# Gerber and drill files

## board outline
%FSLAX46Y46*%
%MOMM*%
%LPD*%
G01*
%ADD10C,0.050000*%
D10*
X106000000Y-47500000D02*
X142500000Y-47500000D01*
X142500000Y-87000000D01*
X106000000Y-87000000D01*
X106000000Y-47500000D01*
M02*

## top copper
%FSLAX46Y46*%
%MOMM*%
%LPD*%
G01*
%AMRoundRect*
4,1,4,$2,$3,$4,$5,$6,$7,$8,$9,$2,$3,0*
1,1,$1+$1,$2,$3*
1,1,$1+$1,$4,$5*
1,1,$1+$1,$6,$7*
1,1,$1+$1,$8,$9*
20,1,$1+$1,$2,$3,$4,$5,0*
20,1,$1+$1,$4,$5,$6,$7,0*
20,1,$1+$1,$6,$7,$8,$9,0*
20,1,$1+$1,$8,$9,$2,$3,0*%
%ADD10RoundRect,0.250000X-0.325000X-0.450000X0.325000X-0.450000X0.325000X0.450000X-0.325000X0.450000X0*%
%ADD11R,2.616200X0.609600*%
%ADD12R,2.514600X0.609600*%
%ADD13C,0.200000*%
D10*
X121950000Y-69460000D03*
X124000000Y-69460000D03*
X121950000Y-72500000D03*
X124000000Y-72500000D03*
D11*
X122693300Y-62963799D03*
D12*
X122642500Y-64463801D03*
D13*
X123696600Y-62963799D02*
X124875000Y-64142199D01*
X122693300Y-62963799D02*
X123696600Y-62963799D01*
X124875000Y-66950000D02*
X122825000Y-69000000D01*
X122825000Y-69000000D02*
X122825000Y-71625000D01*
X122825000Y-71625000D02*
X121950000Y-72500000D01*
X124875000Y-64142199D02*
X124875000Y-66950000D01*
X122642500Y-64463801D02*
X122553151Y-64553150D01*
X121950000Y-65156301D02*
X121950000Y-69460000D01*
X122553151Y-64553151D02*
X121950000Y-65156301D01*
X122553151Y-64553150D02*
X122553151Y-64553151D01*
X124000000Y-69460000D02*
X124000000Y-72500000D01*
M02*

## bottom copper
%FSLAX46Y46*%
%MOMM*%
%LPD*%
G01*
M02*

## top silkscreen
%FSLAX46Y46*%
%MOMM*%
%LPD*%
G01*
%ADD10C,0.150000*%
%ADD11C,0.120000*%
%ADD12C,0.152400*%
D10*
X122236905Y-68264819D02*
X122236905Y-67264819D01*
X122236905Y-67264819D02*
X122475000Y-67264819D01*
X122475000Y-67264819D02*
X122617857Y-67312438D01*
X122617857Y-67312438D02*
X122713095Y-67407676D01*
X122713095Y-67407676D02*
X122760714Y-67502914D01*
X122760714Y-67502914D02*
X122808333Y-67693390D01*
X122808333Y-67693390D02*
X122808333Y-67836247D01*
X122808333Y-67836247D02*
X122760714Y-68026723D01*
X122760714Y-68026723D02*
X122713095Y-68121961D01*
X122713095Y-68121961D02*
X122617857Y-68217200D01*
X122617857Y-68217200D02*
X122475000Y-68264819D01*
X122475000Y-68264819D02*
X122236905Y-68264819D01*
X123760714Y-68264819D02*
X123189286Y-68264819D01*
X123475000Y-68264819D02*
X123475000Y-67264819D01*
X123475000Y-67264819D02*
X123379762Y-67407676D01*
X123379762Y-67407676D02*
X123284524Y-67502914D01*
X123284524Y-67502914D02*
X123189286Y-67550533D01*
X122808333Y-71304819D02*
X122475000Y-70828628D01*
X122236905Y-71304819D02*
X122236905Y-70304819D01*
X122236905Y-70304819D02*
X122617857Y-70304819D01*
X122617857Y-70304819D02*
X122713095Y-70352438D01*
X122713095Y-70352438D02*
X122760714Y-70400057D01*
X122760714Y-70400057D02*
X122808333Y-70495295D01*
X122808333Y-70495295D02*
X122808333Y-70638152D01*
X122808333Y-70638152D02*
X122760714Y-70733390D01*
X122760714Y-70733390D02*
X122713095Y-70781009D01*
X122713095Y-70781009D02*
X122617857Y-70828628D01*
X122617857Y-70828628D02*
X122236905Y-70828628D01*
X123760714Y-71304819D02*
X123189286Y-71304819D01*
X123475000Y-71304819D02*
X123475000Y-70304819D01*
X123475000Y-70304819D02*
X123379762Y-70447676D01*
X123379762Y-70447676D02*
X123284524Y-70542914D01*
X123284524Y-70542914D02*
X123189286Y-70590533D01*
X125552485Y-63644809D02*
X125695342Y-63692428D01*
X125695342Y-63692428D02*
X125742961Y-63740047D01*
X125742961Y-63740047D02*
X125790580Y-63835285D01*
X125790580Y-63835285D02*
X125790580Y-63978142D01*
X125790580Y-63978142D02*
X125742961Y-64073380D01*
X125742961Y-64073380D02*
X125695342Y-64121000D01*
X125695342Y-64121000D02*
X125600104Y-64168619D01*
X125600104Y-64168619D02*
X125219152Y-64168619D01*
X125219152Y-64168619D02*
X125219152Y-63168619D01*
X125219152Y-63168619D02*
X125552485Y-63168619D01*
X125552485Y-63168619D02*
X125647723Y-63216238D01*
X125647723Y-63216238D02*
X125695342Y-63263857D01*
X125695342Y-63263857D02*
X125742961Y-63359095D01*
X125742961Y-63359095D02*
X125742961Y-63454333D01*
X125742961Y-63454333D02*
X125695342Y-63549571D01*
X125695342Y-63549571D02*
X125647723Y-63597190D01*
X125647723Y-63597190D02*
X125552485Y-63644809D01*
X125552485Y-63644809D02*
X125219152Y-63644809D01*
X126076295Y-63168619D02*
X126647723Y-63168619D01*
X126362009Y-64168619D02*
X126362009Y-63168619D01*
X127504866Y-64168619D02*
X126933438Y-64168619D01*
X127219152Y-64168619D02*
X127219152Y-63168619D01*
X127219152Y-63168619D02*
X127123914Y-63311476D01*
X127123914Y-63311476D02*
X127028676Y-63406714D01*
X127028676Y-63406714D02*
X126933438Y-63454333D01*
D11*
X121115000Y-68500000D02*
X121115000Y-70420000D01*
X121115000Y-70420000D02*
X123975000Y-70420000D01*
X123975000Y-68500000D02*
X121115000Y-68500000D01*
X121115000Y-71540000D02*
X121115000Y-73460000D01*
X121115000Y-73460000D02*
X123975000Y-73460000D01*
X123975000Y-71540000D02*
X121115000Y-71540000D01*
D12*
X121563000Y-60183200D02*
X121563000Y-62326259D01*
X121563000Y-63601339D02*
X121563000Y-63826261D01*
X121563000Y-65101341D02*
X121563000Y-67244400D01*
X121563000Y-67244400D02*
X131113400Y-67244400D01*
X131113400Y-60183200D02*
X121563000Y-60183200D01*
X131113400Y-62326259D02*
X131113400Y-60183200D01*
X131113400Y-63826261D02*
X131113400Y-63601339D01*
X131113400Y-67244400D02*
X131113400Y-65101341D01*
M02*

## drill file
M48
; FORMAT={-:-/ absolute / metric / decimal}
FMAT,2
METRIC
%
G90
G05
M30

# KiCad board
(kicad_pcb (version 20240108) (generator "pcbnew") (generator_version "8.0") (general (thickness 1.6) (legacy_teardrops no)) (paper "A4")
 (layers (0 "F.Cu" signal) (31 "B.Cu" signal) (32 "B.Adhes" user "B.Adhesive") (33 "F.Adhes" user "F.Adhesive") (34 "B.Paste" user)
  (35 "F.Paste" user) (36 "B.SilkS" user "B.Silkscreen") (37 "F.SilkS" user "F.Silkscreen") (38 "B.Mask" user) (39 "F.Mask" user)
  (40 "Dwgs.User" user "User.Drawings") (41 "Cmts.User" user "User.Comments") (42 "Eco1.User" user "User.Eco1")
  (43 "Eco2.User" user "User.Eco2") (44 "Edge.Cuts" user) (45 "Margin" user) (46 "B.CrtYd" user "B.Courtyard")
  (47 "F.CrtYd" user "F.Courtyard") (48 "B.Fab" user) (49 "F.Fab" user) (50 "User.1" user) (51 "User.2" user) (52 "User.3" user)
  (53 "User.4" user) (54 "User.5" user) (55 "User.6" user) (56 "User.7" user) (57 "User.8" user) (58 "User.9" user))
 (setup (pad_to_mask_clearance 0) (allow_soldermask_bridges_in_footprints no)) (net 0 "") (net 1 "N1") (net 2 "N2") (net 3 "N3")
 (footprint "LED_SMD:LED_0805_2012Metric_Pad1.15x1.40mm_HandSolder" (layer "F.Cu") (at 122.975 69.46)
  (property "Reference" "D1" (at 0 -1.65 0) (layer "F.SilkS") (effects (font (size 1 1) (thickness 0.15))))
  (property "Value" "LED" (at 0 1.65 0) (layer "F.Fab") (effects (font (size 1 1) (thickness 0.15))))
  (fp_line (start -1.86 -0.96) (end -1.86 0.96) (stroke (width 0.12) (type solid)) (layer "F.SilkS"))
  (fp_line (start -1.86 0.96) (end 1 0.96) (stroke (width 0.12) (type solid)) (layer "F.SilkS"))
  (fp_line (start 1 -0.96) (end -1.86 -0.96) (stroke (width 0.12) (type solid)) (layer "F.SilkS"))
  (pad "1" smd roundrect (at -1.025 0) (size 1.15 1.4) (layers "F.Cu" "F.Paste" "F.Mask") (roundrect_rratio 0.217391) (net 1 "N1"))
  (pad "2" smd roundrect (at 1.025 0) (size 1.15 1.4) (layers "F.Cu" "F.Paste" "F.Mask") (roundrect_rratio 0.217391) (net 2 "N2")))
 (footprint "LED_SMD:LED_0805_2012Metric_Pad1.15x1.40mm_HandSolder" (layer "F.Cu") (at 122.975 72.5)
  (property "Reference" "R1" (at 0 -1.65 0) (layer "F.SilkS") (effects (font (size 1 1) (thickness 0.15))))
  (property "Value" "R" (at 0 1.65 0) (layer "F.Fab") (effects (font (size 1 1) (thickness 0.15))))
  (fp_line (start -1.86 -0.96) (end -1.86 0.96) (stroke (width 0.12) (type solid)) (layer "F.SilkS"))
  (fp_line (start -1.86 0.96) (end 1 0.96) (stroke (width 0.12) (type solid)) (layer "F.SilkS"))
  (fp_line (start 1 -0.96) (end -1.86 -0.96) (stroke (width 0.12) (type solid)) (layer "F.SilkS"))
  (pad "1" smd roundrect (at -1.025 0) (size 1.15 1.4) (layers "F.Cu" "F.Paste" "F.Mask") (roundrect_rratio 0.217391) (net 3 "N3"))
  (pad "2" smd roundrect (at 1.025 0) (size 1.15 1.4) (layers "F.Cu" "F.Paste" "F.Mask") (roundrect_rratio 0.217391) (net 2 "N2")))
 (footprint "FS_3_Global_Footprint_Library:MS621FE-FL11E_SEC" (layer "F.Cu") (at 126.3382 63.7138)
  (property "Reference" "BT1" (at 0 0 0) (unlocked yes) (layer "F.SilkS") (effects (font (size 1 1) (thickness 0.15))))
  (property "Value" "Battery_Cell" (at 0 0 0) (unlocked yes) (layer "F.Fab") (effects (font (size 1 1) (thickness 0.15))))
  (fp_line (start -4.7752 -3.5306) (end -4.7752 -1.387541) (stroke (width 0.1524) (type solid)) (layer "F.SilkS"))
  (fp_line (start -4.7752 -0.112461) (end -4.7752 0.112461) (stroke (width 0.1524) (type solid)) (layer "F.SilkS"))
  (fp_line (start -4.7752 1.387541) (end -4.7752 3.5306) (stroke (width 0.1524) (type solid)) (layer "F.SilkS"))
  (fp_line (start -4.7752 3.5306) (end 4.7752 3.5306) (stroke (width 0.1524) (type solid)) (layer "F.SilkS"))
  (fp_line (start 4.7752 -3.5306) (end -4.7752 -3.5306) (stroke (width 0.1524) (type solid)) (layer "F.SilkS"))
  (fp_line (start 4.7752 -1.387541) (end 4.7752 -3.5306) (stroke (width 0.1524) (type solid)) (layer "F.SilkS"))
  (fp_line (start 4.7752 0.112461) (end 4.7752 -0.112461) (stroke (width 0.1524) (type solid)) (layer "F.SilkS"))
  (fp_line (start 4.7752 3.5306) (end 4.7752 1.387541) (stroke (width 0.1524) (type solid)) (layer "F.SilkS"))
  (pad "1" smd rect (at -3.6449 -0.750001) (size 2.6162 0.6096) (layers "F.Cu" "F.Paste" "F.Mask") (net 3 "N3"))
  (pad "2" smd rect (at -3.6957 0.750001) (size 2.5146 0.6096) (layers "F.Cu" "F.Paste" "F.Mask") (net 1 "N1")))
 (gr_rect (start 106 47.5) (end 142.5 87) (stroke (width 0.05) (type default)) (fill none) (layer "Edge.Cuts"))
 (segment (start 123.6966 62.963799) (end 124.875 64.142199) (width 0.2) (layer "F.Cu") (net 3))
 (segment (start 122.6933 62.963799) (end 123.6966 62.963799) (width 0.2) (layer "F.Cu") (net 3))
 (segment (start 124.875 66.95) (end 122.825 69) (width 0.2) (layer "F.Cu") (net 3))
 (segment (start 122.825 69) (end 122.825 71.625) (width 0.2) (layer "F.Cu") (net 3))
 (segment (start 122.825 71.625) (end 121.95 72.5) (width 0.2) (layer "F.Cu") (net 3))
 (segment (start 124.875 64.142199) (end 124.875 66.95) (width 0.2) (layer "F.Cu") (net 3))
 (segment (start 122.6425 64.463801) (end 122.553151 64.55315) (width 0.2) (layer "F.Cu") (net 1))
 (segment (start 121.95 65.156301) (end 121.95 69.46) (width 0.2) (layer "F.Cu") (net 1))
 (segment (start 122.553151 64.553151) (end 121.95 65.156301) (width 0.2) (layer "F.Cu") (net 1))
 (segment (start 122.553151 64.55315) (end 122.553151 64.553151) (width 0.2) (layer "F.Cu") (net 1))
 (segment (start 124 69.46) (end 124 72.5) (width 0.2) (layer "F.Cu") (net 2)))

